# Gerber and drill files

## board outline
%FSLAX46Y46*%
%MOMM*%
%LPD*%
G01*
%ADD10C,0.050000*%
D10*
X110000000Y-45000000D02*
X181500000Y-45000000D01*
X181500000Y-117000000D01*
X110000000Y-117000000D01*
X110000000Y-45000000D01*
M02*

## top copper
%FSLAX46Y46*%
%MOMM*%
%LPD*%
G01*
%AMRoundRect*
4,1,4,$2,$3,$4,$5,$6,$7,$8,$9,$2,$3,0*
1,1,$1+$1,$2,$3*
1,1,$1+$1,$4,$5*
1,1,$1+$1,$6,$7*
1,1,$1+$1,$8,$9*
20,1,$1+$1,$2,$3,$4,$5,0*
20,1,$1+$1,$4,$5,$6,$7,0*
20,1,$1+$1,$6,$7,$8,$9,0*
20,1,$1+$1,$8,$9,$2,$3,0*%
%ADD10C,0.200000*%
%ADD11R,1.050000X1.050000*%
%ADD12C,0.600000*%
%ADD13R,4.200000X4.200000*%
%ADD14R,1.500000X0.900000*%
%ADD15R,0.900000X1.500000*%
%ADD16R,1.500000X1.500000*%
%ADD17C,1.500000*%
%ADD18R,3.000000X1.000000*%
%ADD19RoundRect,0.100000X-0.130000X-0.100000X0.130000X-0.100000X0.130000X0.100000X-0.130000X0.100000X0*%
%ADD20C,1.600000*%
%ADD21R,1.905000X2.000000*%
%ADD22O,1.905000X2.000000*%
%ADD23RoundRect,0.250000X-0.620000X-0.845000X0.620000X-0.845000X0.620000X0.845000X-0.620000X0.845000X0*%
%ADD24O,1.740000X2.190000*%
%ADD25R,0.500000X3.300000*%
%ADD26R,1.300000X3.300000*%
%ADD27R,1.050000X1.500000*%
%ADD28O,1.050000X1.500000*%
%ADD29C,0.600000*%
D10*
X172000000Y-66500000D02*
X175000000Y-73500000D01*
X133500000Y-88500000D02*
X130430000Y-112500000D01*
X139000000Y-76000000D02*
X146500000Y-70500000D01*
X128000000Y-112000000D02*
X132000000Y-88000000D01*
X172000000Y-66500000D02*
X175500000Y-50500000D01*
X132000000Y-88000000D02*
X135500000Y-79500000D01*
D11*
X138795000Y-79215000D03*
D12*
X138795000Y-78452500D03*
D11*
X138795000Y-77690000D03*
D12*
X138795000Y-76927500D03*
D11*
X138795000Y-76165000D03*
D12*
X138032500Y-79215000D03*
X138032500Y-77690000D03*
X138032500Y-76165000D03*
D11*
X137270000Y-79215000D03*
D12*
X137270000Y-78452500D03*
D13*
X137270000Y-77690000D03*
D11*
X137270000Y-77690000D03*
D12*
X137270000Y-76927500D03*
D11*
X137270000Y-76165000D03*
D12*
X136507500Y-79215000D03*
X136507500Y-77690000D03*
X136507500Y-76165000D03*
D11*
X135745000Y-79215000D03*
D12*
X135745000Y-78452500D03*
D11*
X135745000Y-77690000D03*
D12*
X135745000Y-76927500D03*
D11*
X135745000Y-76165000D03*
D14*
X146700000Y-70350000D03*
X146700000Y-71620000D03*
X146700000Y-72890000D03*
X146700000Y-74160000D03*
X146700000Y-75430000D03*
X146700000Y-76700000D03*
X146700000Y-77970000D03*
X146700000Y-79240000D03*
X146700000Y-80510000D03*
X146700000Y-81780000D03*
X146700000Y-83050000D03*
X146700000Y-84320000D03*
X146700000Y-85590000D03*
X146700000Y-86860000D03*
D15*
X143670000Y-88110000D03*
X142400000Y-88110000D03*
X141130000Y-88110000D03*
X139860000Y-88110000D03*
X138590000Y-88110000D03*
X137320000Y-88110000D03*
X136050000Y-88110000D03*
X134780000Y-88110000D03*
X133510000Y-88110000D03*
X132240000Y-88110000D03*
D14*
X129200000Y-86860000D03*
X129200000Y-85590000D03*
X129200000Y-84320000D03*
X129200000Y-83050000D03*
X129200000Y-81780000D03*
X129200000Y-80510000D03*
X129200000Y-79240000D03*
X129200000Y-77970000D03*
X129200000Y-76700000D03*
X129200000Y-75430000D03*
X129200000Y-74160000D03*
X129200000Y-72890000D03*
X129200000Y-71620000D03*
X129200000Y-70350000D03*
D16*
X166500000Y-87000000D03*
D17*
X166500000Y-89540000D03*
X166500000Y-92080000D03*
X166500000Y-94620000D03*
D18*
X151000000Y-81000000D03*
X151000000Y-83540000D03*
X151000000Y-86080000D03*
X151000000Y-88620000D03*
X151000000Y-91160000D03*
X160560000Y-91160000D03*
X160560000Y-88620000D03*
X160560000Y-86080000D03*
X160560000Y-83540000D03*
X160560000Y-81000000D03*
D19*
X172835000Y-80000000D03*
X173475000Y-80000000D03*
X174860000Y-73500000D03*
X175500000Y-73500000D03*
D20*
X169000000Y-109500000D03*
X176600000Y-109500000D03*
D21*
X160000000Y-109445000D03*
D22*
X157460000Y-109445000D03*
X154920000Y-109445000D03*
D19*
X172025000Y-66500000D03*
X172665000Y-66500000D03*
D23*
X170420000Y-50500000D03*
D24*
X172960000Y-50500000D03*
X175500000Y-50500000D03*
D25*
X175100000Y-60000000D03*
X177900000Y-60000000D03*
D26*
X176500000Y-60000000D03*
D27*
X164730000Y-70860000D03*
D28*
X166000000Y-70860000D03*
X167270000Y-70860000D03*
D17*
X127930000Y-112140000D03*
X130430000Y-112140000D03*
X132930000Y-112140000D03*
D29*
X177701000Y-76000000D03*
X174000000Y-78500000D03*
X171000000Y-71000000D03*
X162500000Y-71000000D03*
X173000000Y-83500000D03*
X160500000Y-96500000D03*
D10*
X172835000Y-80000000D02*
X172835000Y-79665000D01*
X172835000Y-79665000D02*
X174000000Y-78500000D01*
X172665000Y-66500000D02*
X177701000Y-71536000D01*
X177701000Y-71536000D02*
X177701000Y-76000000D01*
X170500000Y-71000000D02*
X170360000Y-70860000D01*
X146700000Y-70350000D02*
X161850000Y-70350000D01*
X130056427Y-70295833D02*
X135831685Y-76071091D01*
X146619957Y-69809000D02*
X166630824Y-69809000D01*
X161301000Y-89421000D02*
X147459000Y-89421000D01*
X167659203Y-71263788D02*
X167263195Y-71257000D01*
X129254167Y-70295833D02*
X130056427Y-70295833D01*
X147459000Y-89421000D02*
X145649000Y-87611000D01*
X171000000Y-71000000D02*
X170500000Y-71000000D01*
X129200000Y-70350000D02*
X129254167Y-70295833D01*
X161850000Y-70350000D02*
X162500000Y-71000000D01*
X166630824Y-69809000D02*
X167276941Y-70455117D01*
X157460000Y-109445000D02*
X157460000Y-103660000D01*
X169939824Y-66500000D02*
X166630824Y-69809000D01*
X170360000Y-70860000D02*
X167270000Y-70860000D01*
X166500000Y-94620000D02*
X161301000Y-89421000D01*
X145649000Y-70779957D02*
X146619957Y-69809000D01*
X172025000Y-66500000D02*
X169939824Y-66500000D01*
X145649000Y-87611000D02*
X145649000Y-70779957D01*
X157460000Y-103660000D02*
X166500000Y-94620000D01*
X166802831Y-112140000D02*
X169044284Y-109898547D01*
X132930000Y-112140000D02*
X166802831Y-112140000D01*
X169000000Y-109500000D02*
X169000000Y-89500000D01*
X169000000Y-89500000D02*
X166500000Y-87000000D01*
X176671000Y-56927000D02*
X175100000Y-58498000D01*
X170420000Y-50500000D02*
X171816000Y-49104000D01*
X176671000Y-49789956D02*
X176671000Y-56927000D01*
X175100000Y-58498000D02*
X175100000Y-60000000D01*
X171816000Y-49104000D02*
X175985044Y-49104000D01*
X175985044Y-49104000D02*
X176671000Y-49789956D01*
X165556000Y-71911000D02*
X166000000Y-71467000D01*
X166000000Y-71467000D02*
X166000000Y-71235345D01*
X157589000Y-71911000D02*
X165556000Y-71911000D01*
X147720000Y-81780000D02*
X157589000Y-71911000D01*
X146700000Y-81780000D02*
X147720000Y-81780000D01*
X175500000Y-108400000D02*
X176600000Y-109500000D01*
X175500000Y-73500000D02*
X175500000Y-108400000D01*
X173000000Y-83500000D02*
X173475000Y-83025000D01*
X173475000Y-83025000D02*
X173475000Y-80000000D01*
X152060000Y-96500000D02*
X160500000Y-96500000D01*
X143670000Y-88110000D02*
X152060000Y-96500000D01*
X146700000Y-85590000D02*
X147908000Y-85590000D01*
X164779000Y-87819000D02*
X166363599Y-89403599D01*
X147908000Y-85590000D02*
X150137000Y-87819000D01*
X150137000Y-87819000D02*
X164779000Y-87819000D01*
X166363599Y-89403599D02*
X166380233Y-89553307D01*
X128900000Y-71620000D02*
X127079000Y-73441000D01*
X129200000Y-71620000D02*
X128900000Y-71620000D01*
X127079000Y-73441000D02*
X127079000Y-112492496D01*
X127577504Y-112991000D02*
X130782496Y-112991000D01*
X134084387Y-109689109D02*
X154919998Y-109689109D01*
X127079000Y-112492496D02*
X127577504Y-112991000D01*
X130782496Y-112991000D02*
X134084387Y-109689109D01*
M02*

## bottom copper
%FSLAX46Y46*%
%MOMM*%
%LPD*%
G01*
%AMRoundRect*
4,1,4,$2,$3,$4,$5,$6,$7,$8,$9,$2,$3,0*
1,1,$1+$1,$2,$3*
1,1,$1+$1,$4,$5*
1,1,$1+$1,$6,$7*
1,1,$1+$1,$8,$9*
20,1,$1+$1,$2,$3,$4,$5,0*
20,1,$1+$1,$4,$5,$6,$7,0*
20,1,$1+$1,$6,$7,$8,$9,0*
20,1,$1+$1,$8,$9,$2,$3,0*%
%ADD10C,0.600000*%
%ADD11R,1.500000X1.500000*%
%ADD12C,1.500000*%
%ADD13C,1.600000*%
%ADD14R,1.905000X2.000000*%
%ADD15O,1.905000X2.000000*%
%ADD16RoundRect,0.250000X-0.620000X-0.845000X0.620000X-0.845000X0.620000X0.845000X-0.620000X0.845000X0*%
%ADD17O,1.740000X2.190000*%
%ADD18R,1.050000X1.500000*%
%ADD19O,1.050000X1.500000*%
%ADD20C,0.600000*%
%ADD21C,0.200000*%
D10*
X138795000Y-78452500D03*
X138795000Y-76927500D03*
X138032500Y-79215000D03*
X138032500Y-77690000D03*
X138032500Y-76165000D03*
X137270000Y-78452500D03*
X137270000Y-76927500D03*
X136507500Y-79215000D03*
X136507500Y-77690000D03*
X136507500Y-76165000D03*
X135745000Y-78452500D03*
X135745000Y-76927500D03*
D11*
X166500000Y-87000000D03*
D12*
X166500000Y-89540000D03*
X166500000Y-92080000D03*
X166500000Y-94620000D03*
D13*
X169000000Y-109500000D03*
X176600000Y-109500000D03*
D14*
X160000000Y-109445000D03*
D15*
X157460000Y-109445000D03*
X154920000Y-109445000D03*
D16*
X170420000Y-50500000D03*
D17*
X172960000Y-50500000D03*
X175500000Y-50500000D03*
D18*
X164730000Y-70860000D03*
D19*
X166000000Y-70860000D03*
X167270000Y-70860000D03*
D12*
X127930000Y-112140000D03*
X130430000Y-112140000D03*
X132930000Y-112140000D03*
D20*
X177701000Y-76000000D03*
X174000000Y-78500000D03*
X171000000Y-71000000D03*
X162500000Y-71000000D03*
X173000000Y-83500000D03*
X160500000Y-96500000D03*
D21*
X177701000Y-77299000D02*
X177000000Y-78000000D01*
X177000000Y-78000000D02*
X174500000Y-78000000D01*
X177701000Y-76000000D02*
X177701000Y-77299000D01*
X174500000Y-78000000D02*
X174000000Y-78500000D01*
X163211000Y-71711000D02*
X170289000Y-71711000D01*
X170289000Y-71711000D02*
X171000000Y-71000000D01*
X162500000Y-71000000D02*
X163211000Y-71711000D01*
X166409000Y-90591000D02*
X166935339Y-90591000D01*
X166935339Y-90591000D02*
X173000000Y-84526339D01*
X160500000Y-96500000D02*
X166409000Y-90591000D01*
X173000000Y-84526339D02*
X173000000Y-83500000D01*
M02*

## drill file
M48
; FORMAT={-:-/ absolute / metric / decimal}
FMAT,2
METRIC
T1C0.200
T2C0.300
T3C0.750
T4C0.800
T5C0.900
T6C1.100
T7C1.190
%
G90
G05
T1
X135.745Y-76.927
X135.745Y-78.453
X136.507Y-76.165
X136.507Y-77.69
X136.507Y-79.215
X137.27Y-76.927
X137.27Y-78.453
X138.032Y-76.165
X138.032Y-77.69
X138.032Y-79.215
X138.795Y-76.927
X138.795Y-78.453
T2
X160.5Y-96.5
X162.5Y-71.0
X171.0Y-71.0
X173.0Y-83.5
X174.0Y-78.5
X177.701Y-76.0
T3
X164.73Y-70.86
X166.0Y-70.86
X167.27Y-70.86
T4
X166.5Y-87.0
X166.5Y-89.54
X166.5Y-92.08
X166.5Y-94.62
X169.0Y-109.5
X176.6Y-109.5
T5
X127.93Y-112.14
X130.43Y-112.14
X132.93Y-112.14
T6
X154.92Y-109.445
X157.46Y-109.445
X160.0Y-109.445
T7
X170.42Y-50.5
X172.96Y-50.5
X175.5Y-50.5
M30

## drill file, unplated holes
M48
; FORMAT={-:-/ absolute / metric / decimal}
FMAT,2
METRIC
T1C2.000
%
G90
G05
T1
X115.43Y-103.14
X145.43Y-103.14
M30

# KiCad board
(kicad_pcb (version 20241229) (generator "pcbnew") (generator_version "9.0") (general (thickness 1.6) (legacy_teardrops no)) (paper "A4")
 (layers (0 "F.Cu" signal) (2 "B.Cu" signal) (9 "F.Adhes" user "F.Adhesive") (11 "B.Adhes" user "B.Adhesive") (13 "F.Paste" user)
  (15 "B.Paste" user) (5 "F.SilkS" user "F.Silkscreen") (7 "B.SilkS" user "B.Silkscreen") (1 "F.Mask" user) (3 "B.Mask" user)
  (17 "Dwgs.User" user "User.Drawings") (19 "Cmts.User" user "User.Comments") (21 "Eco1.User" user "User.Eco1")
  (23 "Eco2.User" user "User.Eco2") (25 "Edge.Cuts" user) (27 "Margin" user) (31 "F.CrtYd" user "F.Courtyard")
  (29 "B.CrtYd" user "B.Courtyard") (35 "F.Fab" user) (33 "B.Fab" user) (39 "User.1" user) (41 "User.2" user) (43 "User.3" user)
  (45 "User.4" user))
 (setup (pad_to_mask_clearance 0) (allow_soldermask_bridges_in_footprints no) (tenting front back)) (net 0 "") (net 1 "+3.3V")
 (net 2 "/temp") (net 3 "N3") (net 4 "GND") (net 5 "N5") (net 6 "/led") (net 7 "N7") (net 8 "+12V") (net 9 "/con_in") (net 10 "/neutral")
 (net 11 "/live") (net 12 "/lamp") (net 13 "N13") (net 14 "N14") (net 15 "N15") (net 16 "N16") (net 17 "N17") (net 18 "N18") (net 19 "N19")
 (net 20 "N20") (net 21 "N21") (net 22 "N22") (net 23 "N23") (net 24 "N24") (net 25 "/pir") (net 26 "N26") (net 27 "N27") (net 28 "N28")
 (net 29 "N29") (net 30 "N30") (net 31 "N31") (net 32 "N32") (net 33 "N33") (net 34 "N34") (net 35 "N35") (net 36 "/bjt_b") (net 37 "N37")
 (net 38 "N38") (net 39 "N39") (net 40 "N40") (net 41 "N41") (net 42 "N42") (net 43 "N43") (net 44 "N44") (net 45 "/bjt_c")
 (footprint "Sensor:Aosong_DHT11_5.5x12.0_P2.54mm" (layer "F.Cu") (at 166.5 87)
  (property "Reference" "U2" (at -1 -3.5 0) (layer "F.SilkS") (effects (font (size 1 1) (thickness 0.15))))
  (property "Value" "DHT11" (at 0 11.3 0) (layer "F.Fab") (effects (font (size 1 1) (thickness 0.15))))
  (pad "1" thru_hole rect (at 0 0) (size 1.5 1.5) (drill 0.8) (layers "*.Cu" "*.Mask") (remove_unused_layers no) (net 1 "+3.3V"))
  (pad "2" thru_hole circle (at 0 2.54) (size 1.5 1.5) (drill 0.8) (layers "*.Cu" "*.Mask") (remove_unused_layers no) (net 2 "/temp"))
  (pad "3" thru_hole circle (at 0 5.08) (size 1.5 1.5) (drill 0.8) (layers "*.Cu" "*.Mask") (remove_unused_layers no) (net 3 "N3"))
  (pad "4" thru_hole circle (at 0 7.62) (size 1.5 1.5) (drill 0.8) (layers "*.Cu" "*.Mask") (remove_unused_layers no) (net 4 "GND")))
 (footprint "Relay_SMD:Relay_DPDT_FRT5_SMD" (layer "F.Cu") (at 155.78 86.08)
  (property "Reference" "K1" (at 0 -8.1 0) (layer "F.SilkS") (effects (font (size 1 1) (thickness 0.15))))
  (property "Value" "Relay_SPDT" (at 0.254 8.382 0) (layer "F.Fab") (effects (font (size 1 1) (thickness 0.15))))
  (pad "1" smd rect (at -4.78 -5.08) (size 3 1) (layers "F.Cu" "F.Mask" "F.Paste"))
  (pad "2" smd rect (at -4.78 -2.54) (size 3 1) (layers "F.Cu" "F.Mask" "F.Paste"))
  (pad "3" smd rect (at -4.78 0) (size 3 1) (layers "F.Cu" "F.Mask" "F.Paste"))
  (pad "4" smd rect (at -4.78 2.54) (size 3 1) (layers "F.Cu" "F.Mask" "F.Paste"))
  (pad "5" smd rect (at -4.78 5.08) (size 3 1) (layers "F.Cu" "F.Mask" "F.Paste"))
  (pad "6" smd rect (at 4.78 5.08) (size 3 1) (layers "F.Cu" "F.Mask" "F.Paste"))
  (pad "7" smd rect (at 4.78 2.54) (size 3 1) (layers "F.Cu" "F.Mask" "F.Paste"))
  (pad "8" smd rect (at 4.78 0) (size 3 1) (layers "F.Cu" "F.Mask" "F.Paste"))
  (pad "9" smd rect (at 4.78 -2.54) (size 3 1) (layers "F.Cu" "F.Mask" "F.Paste"))
  (pad "10" smd rect (at 4.78 -5.08) (size 3 1) (layers "F.Cu" "F.Mask" "F.Paste")))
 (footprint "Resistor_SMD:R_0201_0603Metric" (layer "F.Cu") (at 173.155 80)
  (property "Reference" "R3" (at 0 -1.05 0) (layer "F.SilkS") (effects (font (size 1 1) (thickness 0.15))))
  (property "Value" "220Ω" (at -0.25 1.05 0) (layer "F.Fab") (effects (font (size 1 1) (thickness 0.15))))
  (pad "" smd roundrect (at -0.345 0) (size 0.318 0.36) (layers "F.Paste") (roundrect_rratio 0.25))
  (pad "" smd roundrect (at 0.345 0) (size 0.318 0.36) (layers "F.Paste") (roundrect_rratio 0.25))
  (pad "1" smd roundrect (at -0.32 0) (size 0.46 0.4) (layers "F.Cu" "F.Mask") (roundrect_rratio 0.25) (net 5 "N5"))
  (pad "2" smd roundrect (at 0.32 0) (size 0.46 0.4) (layers "F.Cu" "F.Mask") (roundrect_rratio 0.25) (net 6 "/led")))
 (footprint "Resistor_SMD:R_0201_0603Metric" (layer "F.Cu") (at 175.18 73.5)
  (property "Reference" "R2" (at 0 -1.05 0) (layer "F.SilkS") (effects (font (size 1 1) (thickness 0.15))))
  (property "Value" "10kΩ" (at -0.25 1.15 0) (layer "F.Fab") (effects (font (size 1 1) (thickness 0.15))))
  (pad "" smd roundrect (at -0.345 0) (size 0.318 0.36) (layers "F.Paste") (roundrect_rratio 0.25))
  (pad "" smd roundrect (at 0.345 0) (size 0.318 0.36) (layers "F.Paste") (roundrect_rratio 0.25))
  (pad "1" smd roundrect (at -0.32 0) (size 0.46 0.4) (layers "F.Cu" "F.Mask") (roundrect_rratio 0.25) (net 4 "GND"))
  (pad "2" smd roundrect (at 0.32 0) (size 0.46 0.4) (layers "F.Cu" "F.Mask") (roundrect_rratio 0.25) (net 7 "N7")))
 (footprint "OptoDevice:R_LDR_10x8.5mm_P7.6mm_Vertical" (layer "F.Cu") (at 169 109.5)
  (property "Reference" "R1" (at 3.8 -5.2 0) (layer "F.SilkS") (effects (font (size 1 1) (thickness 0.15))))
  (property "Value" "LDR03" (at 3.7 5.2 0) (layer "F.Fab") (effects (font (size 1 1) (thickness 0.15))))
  (pad "1" thru_hole circle (at 0 0) (size 1.6 1.6) (drill 0.8) (layers "*.Cu" "*.Mask") (remove_unused_layers no) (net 1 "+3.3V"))
  (pad "2" thru_hole circle (at 7.6 0) (size 1.6 1.6) (drill 0.8) (layers "*.Cu" "*.Mask") (remove_unused_layers no) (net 7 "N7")))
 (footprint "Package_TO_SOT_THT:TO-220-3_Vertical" (layer "F.Cu") (at 160 109.445 180)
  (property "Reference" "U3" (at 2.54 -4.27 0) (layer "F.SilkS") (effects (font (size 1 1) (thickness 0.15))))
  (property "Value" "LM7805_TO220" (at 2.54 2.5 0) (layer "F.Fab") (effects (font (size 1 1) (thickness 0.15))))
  (pad "1" thru_hole rect (at 0 0 180) (size 1.905 2) (drill 1.1) (layers "*.Cu" "*.Mask") (remove_unused_layers no) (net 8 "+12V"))
  (pad "2" thru_hole oval (at 2.54 0 180) (size 1.905 2) (drill 1.1) (layers "*.Cu" "*.Mask") (remove_unused_layers no) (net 4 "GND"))
  (pad "3" thru_hole oval (at 5.08 0 180) (size 1.905 2) (drill 1.1) (layers "*.Cu" "*.Mask") (remove_unused_layers no) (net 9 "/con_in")))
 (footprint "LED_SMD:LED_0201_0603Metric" (layer "F.Cu") (at 172.345 66.5)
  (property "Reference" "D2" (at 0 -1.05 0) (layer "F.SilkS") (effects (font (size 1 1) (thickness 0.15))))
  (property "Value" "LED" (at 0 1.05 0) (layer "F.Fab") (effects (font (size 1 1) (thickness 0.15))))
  (pad "" smd roundrect (at -0.345 0) (size 0.318 0.36) (layers "F.Paste") (roundrect_rratio 0.25))
  (pad "" smd roundrect (at 0.345 0) (size 0.318 0.36) (layers "F.Paste") (roundrect_rratio 0.25))
  (pad "1" smd roundrect (at -0.32 0) (size 0.46 0.4) (layers "F.Cu" "F.Mask") (roundrect_rratio 0.25) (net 4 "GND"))
  (pad "2" smd roundrect (at 0.32 0) (size 0.46 0.4) (layers "F.Cu" "F.Mask") (roundrect_rratio 0.25) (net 5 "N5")))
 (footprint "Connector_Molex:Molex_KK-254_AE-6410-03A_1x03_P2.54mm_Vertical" (layer "F.Cu") (at 170.42 50.5)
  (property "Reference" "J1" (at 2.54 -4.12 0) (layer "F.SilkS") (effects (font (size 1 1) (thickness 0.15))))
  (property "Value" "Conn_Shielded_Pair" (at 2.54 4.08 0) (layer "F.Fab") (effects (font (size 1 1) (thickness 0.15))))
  (pad "1" thru_hole roundrect (at 0 0) (size 1.74 2.19) (drill 1.19) (layers "*.Cu" "*.Mask") (remove_unused_layers no)
   (roundrect_rratio 0.143678) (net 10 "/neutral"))
  (pad "2" thru_hole oval (at 2.54 0) (size 1.74 2.19) (drill 1.19) (layers "*.Cu" "*.Mask") (remove_unused_layers no) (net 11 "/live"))
  (pad "3" thru_hole oval (at 5.08 0) (size 1.74 2.19) (drill 1.19) (layers "*.Cu" "*.Mask") (remove_unused_layers no) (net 4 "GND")))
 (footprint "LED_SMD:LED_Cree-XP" (layer "F.Cu") (at 176.5 60)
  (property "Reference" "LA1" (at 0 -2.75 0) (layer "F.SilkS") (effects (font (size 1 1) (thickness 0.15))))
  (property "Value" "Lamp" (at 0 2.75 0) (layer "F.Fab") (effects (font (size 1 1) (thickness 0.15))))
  (pad "" smd rect (at 0 -1) (size 1.01 0.75) (layers "F.Paste"))
  (pad "" smd rect (at 0 0) (size 1.01 0.75) (layers "F.Paste"))
  (pad "" smd rect (at 0 1) (size 1.01 0.75) (layers "F.Paste"))
  (pad "1" smd rect (at -1.4 0) (size 0.5 3.3) (layers "F.Cu" "F.Mask" "F.Paste") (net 10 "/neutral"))
  (pad "2" smd rect (at 1.4 0) (size 0.5 3.3) (layers "F.Cu" "F.Mask" "F.Paste") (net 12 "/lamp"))
  (pad "3" smd rect (at 0 0) (size 1.3 3.3) (layers "F.Cu" "F.Mask")))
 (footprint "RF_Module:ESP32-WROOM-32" (layer "F.Cu") (at 137.95 78.6)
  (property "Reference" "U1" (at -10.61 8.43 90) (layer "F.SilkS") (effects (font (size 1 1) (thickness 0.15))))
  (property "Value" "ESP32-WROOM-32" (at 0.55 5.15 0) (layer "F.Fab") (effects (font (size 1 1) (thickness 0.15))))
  (pad "1" smd rect (at -8.75 -8.25) (size 1.5 0.9) (layers "F.Cu" "F.Mask" "F.Paste") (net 4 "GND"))
  (pad "2" smd rect (at -8.75 -6.98) (size 1.5 0.9) (layers "F.Cu" "F.Mask" "F.Paste") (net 9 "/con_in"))
  (pad "3" smd rect (at -8.75 -5.71) (size 1.5 0.9) (layers "F.Cu" "F.Mask" "F.Paste") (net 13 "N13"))
  (pad "4" smd rect (at -8.75 -4.44) (size 1.5 0.9) (layers "F.Cu" "F.Mask" "F.Paste") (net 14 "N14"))
  (pad "5" smd rect (at -8.75 -3.17) (size 1.5 0.9) (layers "F.Cu" "F.Mask" "F.Paste") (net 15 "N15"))
  (pad "6" smd rect (at -8.75 -1.9) (size 1.5 0.9) (layers "F.Cu" "F.Mask" "F.Paste") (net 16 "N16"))
  (pad "7" smd rect (at -8.75 -0.63) (size 1.5 0.9) (layers "F.Cu" "F.Mask" "F.Paste") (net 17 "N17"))
  (pad "8" smd rect (at -8.75 0.64) (size 1.5 0.9) (layers "F.Cu" "F.Mask" "F.Paste") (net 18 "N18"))
  (pad "9" smd rect (at -8.75 1.91) (size 1.5 0.9) (layers "F.Cu" "F.Mask" "F.Paste") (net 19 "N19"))
  (pad "10" smd rect (at -8.75 3.18) (size 1.5 0.9) (layers "F.Cu" "F.Mask" "F.Paste") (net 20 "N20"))
  (pad "11" smd rect (at -8.75 4.45) (size 1.5 0.9) (layers "F.Cu" "F.Mask" "F.Paste") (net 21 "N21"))
  (pad "12" smd rect (at -8.75 5.72) (size 1.5 0.9) (layers "F.Cu" "F.Mask" "F.Paste") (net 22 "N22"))
  (pad "13" smd rect (at -8.75 6.99) (size 1.5 0.9) (layers "F.Cu" "F.Mask" "F.Paste") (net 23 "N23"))
  (pad "14" smd rect (at -8.75 8.26) (size 1.5 0.9) (layers "F.Cu" "F.Mask" "F.Paste") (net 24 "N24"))
  (pad "15" smd rect (at -5.71 9.51 90) (size 1.5 0.9) (layers "F.Cu" "F.Mask" "F.Paste") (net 4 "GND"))
  (pad "16" smd rect (at -4.44 9.51 90) (size 1.5 0.9) (layers "F.Cu" "F.Mask" "F.Paste") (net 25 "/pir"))
  (pad "17" smd rect (at -3.17 9.51 90) (size 1.5 0.9) (layers "F.Cu" "F.Mask" "F.Paste") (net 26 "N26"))
  (pad "18" smd rect (at -1.9 9.51 90) (size 1.5 0.9) (layers "F.Cu" "F.Mask" "F.Paste") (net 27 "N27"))
  (pad "19" smd rect (at -0.63 9.51 90) (size 1.5 0.9) (layers "F.Cu" "F.Mask" "F.Paste") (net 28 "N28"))
  (pad "20" smd rect (at 0.64 9.51 90) (size 1.5 0.9) (layers "F.Cu" "F.Mask" "F.Paste") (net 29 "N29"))
  (pad "21" smd rect (at 1.91 9.51 90) (size 1.5 0.9) (layers "F.Cu" "F.Mask" "F.Paste") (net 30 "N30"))
  (pad "22" smd rect (at 3.18 9.51 90) (size 1.5 0.9) (layers "F.Cu" "F.Mask" "F.Paste") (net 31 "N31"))
  (pad "23" smd rect (at 4.45 9.51 90) (size 1.5 0.9) (layers "F.Cu" "F.Mask" "F.Paste") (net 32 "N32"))
  (pad "24" smd rect (at 5.72 9.51 90) (size 1.5 0.9) (layers "F.Cu" "F.Mask" "F.Paste") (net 6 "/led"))
  (pad "25" smd rect (at 8.75 8.26) (size 1.5 0.9) (layers "F.Cu" "F.Mask" "F.Paste") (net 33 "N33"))
  (pad "26" smd rect (at 8.75 6.99) (size 1.5 0.9) (layers "F.Cu" "F.Mask" "F.Paste") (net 2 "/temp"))
  (pad "27" smd rect (at 8.75 5.72) (size 1.5 0.9) (layers "F.Cu" "F.Mask" "F.Paste") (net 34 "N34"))
  (pad "28" smd rect (at 8.75 4.45) (size 1.5 0.9) (layers "F.Cu" "F.Mask" "F.Paste") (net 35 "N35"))
  (pad "29" smd rect (at 8.75 3.18) (size 1.5 0.9) (layers "F.Cu" "F.Mask" "F.Paste") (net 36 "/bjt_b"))
  (pad "30" smd rect (at 8.75 1.91) (size 1.5 0.9) (layers "F.Cu" "F.Mask" "F.Paste") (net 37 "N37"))
  (pad "31" smd rect (at 8.75 0.64) (size 1.5 0.9) (layers "F.Cu" "F.Mask" "F.Paste") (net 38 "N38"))
  (pad "32" smd rect (at 8.75 -0.63) (size 1.5 0.9) (layers "F.Cu" "F.Mask" "F.Paste") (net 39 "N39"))
  (pad "33" smd rect (at 8.75 -1.9) (size 1.5 0.9) (layers "F.Cu" "F.Mask" "F.Paste") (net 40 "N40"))
  (pad "34" smd rect (at 8.75 -3.17) (size 1.5 0.9) (layers "F.Cu" "F.Mask" "F.Paste") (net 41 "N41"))
  (pad "35" smd rect (at 8.75 -4.44) (size 1.5 0.9) (layers "F.Cu" "F.Mask" "F.Paste") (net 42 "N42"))
  (pad "36" smd rect (at 8.75 -5.71) (size 1.5 0.9) (layers "F.Cu" "F.Mask" "F.Paste") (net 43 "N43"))
  (pad "37" smd rect (at 8.75 -6.98) (size 1.5 0.9) (layers "F.Cu" "F.Mask" "F.Paste") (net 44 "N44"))
  (pad "38" smd rect (at 8.75 -8.25) (size 1.5 0.9) (layers "F.Cu" "F.Mask" "F.Paste") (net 4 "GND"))
  (pad "39" smd rect (at -2.205 -2.435) (size 1.05 1.05) (layers "F.Cu" "F.Paste") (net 4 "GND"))
  (pad "39" thru_hole circle (at -2.205 -1.6725) (size 0.6 0.6) (drill 0.2) (layers "*.Cu" "F.Mask") (remove_unused_layers no) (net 4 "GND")
   (zone_connect 2))
  (pad "39" smd rect (at -2.205 -0.91) (size 1.05 1.05) (layers "F.Cu" "F.Paste") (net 4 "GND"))
  (pad "39" thru_hole circle (at -2.205 -0.1475) (size 0.6 0.6) (drill 0.2) (layers "*.Cu" "F.Mask") (remove_unused_layers no) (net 4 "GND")
   (zone_connect 2))
  (pad "39" smd rect (at -2.205 0.615) (size 1.05 1.05) (layers "F.Cu" "F.Paste") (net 4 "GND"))
  (pad "39" thru_hole circle (at -1.4425 -2.435) (size 0.6 0.6) (drill 0.2) (layers "*.Cu" "F.Mask") (remove_unused_layers no) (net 4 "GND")
   (zone_connect 2))
  (pad "39" thru_hole circle (at -1.4425 -0.91) (size 0.6 0.6) (drill 0.2) (layers "*.Cu" "F.Mask") (remove_unused_layers no) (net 4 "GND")
   (zone_connect 2))
  (pad "39" thru_hole circle (at -1.4425 0.615) (size 0.6 0.6) (drill 0.2) (layers "*.Cu" "F.Mask") (remove_unused_layers no) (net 4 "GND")
   (zone_connect 2))
  (pad "39" smd rect (at -0.68 -2.435) (size 1.05 1.05) (layers "F.Cu" "F.Paste") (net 4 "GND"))
  (pad "39" thru_hole circle (at -0.68 -1.6725) (size 0.6 0.6) (drill 0.2) (layers "*.Cu" "F.Mask") (remove_unused_layers no) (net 4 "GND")
   (zone_connect 2))
  (pad "39" smd rect (at -0.68 -0.91) (size 1.05 1.05) (layers "F.Cu" "F.Paste") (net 4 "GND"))
  (pad "39" smd rect (at -0.68 -0.91) (size 4.2 4.2) (layers "F.Cu" "F.Mask") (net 4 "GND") (zone_connect 2))
  (pad "39" thru_hole circle (at -0.68 -0.1475) (size 0.6 0.6) (drill 0.2) (layers "*.Cu" "F.Mask") (remove_unused_layers no) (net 4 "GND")
   (zone_connect 2))
  (pad "39" smd rect (at -0.68 0.615) (size 1.05 1.05) (layers "F.Cu" "F.Paste") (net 4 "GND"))
  (pad "39" thru_hole circle (at 0.0825 -2.435) (size 0.6 0.6) (drill 0.2) (layers "*.Cu" "F.Mask") (remove_unused_layers no) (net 4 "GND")
   (zone_connect 2))
  (pad "39" thru_hole circle (at 0.0825 -0.91) (size 0.6 0.6) (drill 0.2) (layers "*.Cu" "F.Mask") (remove_unused_layers no) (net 4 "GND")
   (zone_connect 2))
  (pad "39" thru_hole circle (at 0.0825 0.615) (size 0.6 0.6) (drill 0.2) (layers "*.Cu" "F.Mask") (remove_unused_layers no) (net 4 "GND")
   (zone_connect 2))
  (pad "39" smd rect (at 0.845 -2.435) (size 1.05 1.05) (layers "F.Cu" "F.Paste") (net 4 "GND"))
  (pad "39" thru_hole circle (at 0.845 -1.6725) (size 0.6 0.6) (drill 0.2) (layers "*.Cu" "F.Mask") (remove_unused_layers no) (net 4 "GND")
   (zone_connect 2))
  (pad "39" smd rect (at 0.845 -0.91) (size 1.05 1.05) (layers "F.Cu" "F.Paste") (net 4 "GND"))
  (pad "39" thru_hole circle (at 0.845 -0.1475) (size 0.6 0.6) (drill 0.2) (layers "*.Cu" "F.Mask") (remove_unused_layers no) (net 4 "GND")
   (zone_connect 2))
  (pad "39" smd rect (at 0.845 0.615) (size 1.05 1.05) (layers "F.Cu" "F.Paste") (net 4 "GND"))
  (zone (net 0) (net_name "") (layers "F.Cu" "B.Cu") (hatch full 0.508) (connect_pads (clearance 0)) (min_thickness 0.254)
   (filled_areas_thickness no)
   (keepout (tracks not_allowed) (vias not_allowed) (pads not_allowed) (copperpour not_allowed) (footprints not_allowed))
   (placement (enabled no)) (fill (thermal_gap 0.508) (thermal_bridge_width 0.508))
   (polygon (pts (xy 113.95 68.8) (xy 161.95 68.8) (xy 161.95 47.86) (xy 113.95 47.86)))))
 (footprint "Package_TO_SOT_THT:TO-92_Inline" (layer "F.Cu") (at 164.73 70.86)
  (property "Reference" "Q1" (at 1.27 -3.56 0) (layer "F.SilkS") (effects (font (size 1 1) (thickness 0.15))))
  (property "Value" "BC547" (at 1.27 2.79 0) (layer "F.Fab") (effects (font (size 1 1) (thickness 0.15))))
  (pad "1" thru_hole rect (at 0 0) (size 1.05 1.5) (drill 0.75) (layers "*.Cu" "*.Mask") (remove_unused_layers no) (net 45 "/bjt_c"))
  (pad "2" thru_hole oval (at 1.27 0) (size 1.05 1.5) (drill 0.75) (layers "*.Cu" "*.Mask") (remove_unused_layers no) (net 36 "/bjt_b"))
  (pad "3" thru_hole oval (at 2.54 0) (size 1.05 1.5) (drill 0.75) (layers "*.Cu" "*.Mask") (remove_unused_layers no) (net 4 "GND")))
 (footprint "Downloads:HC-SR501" (layer "F.Cu") (at 130.43 102.14)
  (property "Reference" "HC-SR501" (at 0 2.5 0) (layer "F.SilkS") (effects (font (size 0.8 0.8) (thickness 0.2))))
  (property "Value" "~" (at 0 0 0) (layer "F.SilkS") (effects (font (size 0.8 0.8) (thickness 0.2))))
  (pad "" np_thru_hole circle (at -15 1) (size 2 2) (drill 2) (layers "*.Cu" "*.Mask" "F.SilkS"))
  (pad "" np_thru_hole circle (at 15 1) (size 2 2) (drill 2) (layers "*.Cu" "*.Mask" "F.SilkS"))
  (pad "1" thru_hole circle (at -2.5 10) (size 1.5 1.5) (drill 0.9) (layers "*.Cu" "*.Mask" "F.SilkS") (remove_unused_layers no)
   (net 4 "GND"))
  (pad "2" thru_hole circle (at 0 10) (size 1.5 1.5) (drill 0.9) (layers "*.Cu" "*.Mask" "F.SilkS") (remove_unused_layers no)
   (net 25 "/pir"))
  (pad "3" thru_hole circle (at 2.5 10) (size 1.5 1.5) (drill 0.9) (layers "*.Cu" "*.Mask" "F.SilkS") (remove_unused_layers no)
   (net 1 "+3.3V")))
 (gr_line (start 172 66.5) (end 175 73.5) (stroke (width 0.2) (type default)) (layer "F.Cu") (net 4))
 (gr_line (start 133.5 88.5) (end 130.43 112.5) (stroke (width 0.2) (type default)) (layer "F.Cu") (net 25))
 (gr_line (start 139 76) (end 146.5 70.5) (stroke (width 0.2) (type default)) (layer "F.Cu") (net 4))
 (gr_line (start 128 112) (end 132 88) (stroke (width 0.2) (type default)) (layer "F.Cu") (net 4))
 (gr_line (start 172 66.5) (end 175.5 50.5) (stroke (width 0.2) (type default)) (layer "F.Cu") (net 4))
 (gr_line (start 132 88) (end 135.5 79.5) (stroke (width 0.2) (type default)) (layer "F.Cu") (net 4))
 (gr_rect (start 110 45) (end 181.5 117) (stroke (width 0.05) (type default)) (fill no) (layer "Edge.Cuts"))
 (segment (start 172.835 80) (end 172.835 79.665) (width 0.2) (layer "F.Cu") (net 5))
 (segment (start 172.835 79.665) (end 174 78.5) (width 0.2) (layer "F.Cu") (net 5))
 (segment (start 172.665 66.5) (end 177.701 71.536) (width 0.2) (layer "F.Cu") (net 5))
 (segment (start 177.701 71.536) (end 177.701 76) (width 0.2) (layer "F.Cu") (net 5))
 (via (at 177.701 76) (size 0.6) (drill 0.3) (layers "F.Cu" "B.Cu") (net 5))
 (via (at 174 78.5) (size 0.6) (drill 0.3) (layers "F.Cu" "B.Cu") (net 5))
 (segment (start 177.701 77.299) (end 177 78) (width 0.2) (layer "B.Cu") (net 5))
 (segment (start 177 78) (end 174.5 78) (width 0.2) (layer "B.Cu") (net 5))
 (segment (start 177.701 76) (end 177.701 77.299) (width 0.2) (layer "B.Cu") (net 5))
 (segment (start 174.5 78) (end 174 78.5) (width 0.2) (layer "B.Cu") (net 5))
 (segment (start 170.5 71) (end 170.36 70.86) (width 0.2) (layer "F.Cu") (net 4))
 (segment (start 146.7 70.35) (end 161.85 70.35) (width 0.2) (layer "F.Cu") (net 4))
 (segment (start 130.056427 70.295833) (end 135.831685 76.071091) (width 0.2) (layer "F.Cu") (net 4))
 (segment (start 146.619957 69.809) (end 166.630824 69.809) (width 0.2) (layer "F.Cu") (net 4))
 (segment (start 161.301 89.421) (end 147.459 89.421) (width 0.2) (layer "F.Cu") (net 4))
 (segment (start 167.659203 71.263788) (end 167.263195 71.257) (width 0.2) (layer "F.Cu") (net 4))
 (segment (start 129.254167 70.295833) (end 130.056427 70.295833) (width 0.2) (layer "F.Cu") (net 4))
 (segment (start 147.459 89.421) (end 145.649 87.611) (width 0.2) (layer "F.Cu") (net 4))
 (segment (start 171 71) (end 170.5 71) (width 0.2) (layer "F.Cu") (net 4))
 (segment (start 129.2 70.35) (end 129.254167 70.295833) (width 0.2) (layer "F.Cu") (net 4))
 (segment (start 161.85 70.35) (end 162.5 71) (width 0.2) (layer "F.Cu") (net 4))
 (segment (start 166.630824 69.809) (end 167.276941 70.455117) (width 0.2) (layer "F.Cu") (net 4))
 (segment (start 157.46 109.445) (end 157.46 103.66) (width 0.2) (layer "F.Cu") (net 4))
 (segment (start 169.939824 66.5) (end 166.630824 69.809) (width 0.2) (layer "F.Cu") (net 4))
 (segment (start 170.36 70.86) (end 167.27 70.86) (width 0.2) (layer "F.Cu") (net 4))
 (segment (start 166.5 94.62) (end 161.301 89.421) (width 0.2) (layer "F.Cu") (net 4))
 (segment (start 145.649 70.779957) (end 146.619957 69.809) (width 0.2) (layer "F.Cu") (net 4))
 (segment (start 172.025 66.5) (end 169.939824 66.5) (width 0.2) (layer "F.Cu") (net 4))
 (segment (start 145.649 87.611) (end 145.649 70.779957) (width 0.2) (layer "F.Cu") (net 4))
 (segment (start 157.46 103.66) (end 166.5 94.62) (width 0.2) (layer "F.Cu") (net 4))
 (via (at 171 71) (size 0.6) (drill 0.3) (layers "F.Cu" "B.Cu") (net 4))
 (via (at 162.5 71) (size 0.6) (drill 0.3) (layers "F.Cu" "B.Cu") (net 4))
 (segment (start 163.211 71.711) (end 170.289 71.711) (width 0.2) (layer "B.Cu") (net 4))
 (segment (start 170.289 71.711) (end 171 71) (width 0.2) (layer "B.Cu") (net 4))
 (segment (start 162.5 71) (end 163.211 71.711) (width 0.2) (layer "B.Cu") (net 4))
 (segment (start 166.802831 112.14) (end 169.044284 109.898547) (width 0.2) (layer "F.Cu") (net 1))
 (segment (start 132.93 112.14) (end 166.802831 112.14) (width 0.2) (layer "F.Cu") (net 1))
 (segment (start 169 109.5) (end 169 89.5) (width 0.2) (layer "F.Cu") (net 1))
 (segment (start 169 89.5) (end 166.5 87) (width 0.2) (layer "F.Cu") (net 1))
 (segment (start 176.671 56.927) (end 175.1 58.498) (width 0.2) (layer "F.Cu") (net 10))
 (segment (start 170.42 50.5) (end 171.816 49.104) (width 0.2) (layer "F.Cu") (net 10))
 (segment (start 176.671 49.789956) (end 176.671 56.927) (width 0.2) (layer "F.Cu") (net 10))
 (segment (start 175.1 58.498) (end 175.1 60) (width 0.2) (layer "F.Cu") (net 10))
 (segment (start 171.816 49.104) (end 175.985044 49.104) (width 0.2) (layer "F.Cu") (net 10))
 (segment (start 175.985044 49.104) (end 176.671 49.789956) (width 0.2) (layer "F.Cu") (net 10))
 (segment (start 165.556 71.911) (end 166 71.467) (width 0.2) (layer "F.Cu") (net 36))
 (segment (start 166 71.467) (end 166 71.235345) (width 0.2) (layer "F.Cu") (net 36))
 (segment (start 157.589 71.911) (end 165.556 71.911) (width 0.2) (layer "F.Cu") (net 36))
 (segment (start 147.72 81.78) (end 157.589 71.911) (width 0.2) (layer "F.Cu") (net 36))
 (segment (start 146.7 81.78) (end 147.72 81.78) (width 0.2) (layer "F.Cu") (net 36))
 (segment (start 175.5 108.4) (end 176.6 109.5) (width 0.2) (layer "F.Cu") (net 7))
 (segment (start 175.5 73.5) (end 175.5 108.4) (width 0.2) (layer "F.Cu") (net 7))
 (segment (start 173 83.5) (end 173.475 83.025) (width 0.2) (layer "F.Cu") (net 6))
 (segment (start 173.475 83.025) (end 173.475 80) (width 0.2) (layer "F.Cu") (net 6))
 (segment (start 152.06 96.5) (end 160.5 96.5) (width 0.2) (layer "F.Cu") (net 6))
 (segment (start 143.67 88.11) (end 152.06 96.5) (width 0.2) (layer "F.Cu") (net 6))
 (via (at 173 83.5) (size 0.6) (drill 0.3) (layers "F.Cu" "B.Cu") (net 6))
 (via (at 160.5 96.5) (size 0.6) (drill 0.3) (layers "F.Cu" "B.Cu") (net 6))
 (segment (start 166.409 90.591) (end 166.935339 90.591) (width 0.2) (layer "B.Cu") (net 6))
 (segment (start 166.935339 90.591) (end 173 84.526339) (width 0.2) (layer "B.Cu") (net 6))
 (segment (start 160.5 96.5) (end 166.409 90.591) (width 0.2) (layer "B.Cu") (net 6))
 (segment (start 173 84.526339) (end 173 83.5) (width 0.2) (layer "B.Cu") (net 6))
 (segment (start 146.7 85.59) (end 147.908 85.59) (width 0.2) (layer "F.Cu") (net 2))
 (segment (start 164.779 87.819) (end 166.363599 89.403599) (width 0.2) (layer "F.Cu") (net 2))
 (segment (start 147.908 85.59) (end 150.137 87.819) (width 0.2) (layer "F.Cu") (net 2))
 (segment (start 150.137 87.819) (end 164.779 87.819) (width 0.2) (layer "F.Cu") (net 2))
 (segment (start 166.363599 89.403599) (end 166.380233 89.553307) (width 0.2) (layer "F.Cu") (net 2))
 (segment (start 128.9 71.62) (end 127.079 73.441) (width 0.2) (layer "F.Cu") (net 9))
 (segment (start 129.2 71.62) (end 128.9 71.62) (width 0.2) (layer "F.Cu") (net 9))
 (segment (start 127.079 73.441) (end 127.079 112.492496) (width 0.2) (layer "F.Cu") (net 9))
 (segment (start 127.577504 112.991) (end 130.782496 112.991) (width 0.2) (layer "F.Cu") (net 9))
 (segment (start 134.084387 109.689109) (end 154.919998 109.689109) (width 0.2) (layer "F.Cu") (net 9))
 (segment (start 127.079 112.492496) (end 127.577504 112.991) (width 0.2) (layer "F.Cu") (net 9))
 (segment (start 130.782496 112.991) (end 134.084387 109.689109) (width 0.2) (layer "F.Cu") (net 9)))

